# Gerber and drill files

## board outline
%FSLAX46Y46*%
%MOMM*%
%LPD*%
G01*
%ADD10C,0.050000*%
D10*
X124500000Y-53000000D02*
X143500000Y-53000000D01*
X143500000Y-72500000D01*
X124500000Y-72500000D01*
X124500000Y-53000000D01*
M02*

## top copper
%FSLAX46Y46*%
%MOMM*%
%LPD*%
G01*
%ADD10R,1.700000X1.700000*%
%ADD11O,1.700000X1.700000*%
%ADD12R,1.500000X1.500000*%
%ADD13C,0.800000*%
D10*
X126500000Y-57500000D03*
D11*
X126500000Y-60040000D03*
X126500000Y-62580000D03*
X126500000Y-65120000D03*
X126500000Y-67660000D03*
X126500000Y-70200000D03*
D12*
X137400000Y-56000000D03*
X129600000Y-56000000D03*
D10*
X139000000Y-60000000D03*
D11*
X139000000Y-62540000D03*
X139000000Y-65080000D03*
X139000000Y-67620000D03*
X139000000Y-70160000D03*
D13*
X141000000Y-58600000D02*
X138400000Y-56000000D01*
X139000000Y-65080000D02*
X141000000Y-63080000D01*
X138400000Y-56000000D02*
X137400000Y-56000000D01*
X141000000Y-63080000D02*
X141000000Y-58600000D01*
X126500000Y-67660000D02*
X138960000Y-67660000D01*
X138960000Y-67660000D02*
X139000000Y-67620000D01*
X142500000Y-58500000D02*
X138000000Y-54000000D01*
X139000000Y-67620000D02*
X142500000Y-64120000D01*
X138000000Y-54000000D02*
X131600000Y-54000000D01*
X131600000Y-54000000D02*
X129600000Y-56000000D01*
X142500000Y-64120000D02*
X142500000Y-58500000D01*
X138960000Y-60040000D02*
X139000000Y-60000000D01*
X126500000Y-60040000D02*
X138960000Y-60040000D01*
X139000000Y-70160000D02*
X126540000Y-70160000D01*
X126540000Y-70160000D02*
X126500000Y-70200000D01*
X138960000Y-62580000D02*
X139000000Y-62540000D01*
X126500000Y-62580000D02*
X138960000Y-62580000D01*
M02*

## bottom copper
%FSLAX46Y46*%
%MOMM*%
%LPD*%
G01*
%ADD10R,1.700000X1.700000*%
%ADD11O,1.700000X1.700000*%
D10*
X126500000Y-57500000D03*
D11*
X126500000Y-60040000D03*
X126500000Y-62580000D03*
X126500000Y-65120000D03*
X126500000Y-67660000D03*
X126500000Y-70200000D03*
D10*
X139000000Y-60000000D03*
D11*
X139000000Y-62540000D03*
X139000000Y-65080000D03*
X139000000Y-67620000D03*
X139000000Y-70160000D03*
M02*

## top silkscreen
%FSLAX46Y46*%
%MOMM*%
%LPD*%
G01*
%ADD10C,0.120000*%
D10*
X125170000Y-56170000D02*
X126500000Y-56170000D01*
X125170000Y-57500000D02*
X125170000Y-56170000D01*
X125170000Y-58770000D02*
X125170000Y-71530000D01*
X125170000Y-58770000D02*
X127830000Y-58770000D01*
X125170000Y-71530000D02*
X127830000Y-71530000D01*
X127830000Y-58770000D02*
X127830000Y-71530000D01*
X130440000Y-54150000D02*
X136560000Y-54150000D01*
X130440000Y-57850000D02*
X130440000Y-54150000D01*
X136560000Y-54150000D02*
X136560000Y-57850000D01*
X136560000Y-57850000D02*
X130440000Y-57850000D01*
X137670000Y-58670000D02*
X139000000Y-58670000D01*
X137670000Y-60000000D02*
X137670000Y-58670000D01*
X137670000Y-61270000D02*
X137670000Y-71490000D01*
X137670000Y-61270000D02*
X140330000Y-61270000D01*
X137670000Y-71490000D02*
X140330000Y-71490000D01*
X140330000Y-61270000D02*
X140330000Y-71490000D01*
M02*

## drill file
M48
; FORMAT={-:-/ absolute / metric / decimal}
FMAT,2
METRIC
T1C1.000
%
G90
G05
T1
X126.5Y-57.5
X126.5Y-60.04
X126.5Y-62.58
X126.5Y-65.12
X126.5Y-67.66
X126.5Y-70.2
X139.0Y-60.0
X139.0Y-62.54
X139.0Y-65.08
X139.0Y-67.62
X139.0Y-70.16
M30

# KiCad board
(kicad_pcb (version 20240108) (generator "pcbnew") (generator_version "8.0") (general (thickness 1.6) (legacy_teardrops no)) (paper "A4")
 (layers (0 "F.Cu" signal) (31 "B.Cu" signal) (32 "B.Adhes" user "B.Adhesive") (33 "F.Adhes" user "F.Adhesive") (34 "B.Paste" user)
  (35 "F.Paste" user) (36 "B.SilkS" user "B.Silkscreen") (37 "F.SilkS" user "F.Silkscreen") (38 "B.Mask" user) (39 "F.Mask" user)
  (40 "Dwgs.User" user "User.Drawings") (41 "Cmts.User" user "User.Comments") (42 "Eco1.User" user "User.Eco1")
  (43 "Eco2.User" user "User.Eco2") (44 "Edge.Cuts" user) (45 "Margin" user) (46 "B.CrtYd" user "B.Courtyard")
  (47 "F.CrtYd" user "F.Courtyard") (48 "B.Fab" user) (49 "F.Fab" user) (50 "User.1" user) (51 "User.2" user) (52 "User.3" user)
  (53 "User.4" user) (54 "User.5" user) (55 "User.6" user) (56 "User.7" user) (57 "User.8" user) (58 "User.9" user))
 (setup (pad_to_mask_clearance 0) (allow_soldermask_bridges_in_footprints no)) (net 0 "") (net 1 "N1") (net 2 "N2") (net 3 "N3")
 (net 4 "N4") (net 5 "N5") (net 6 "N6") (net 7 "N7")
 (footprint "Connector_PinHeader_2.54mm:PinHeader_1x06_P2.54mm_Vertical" (layer "F.Cu") (at 126.5 57.5)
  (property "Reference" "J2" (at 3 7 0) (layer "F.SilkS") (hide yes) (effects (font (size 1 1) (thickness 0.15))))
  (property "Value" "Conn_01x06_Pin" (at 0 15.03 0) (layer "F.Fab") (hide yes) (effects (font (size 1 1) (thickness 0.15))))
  (fp_line (start -1.33 -1.33) (end 0 -1.33) (stroke (width 0.12) (type solid)) (layer "F.SilkS"))
  (fp_line (start -1.33 0) (end -1.33 -1.33) (stroke (width 0.12) (type solid)) (layer "F.SilkS"))
  (fp_line (start -1.33 1.27) (end -1.33 14.03) (stroke (width 0.12) (type solid)) (layer "F.SilkS"))
  (fp_line (start -1.33 1.27) (end 1.33 1.27) (stroke (width 0.12) (type solid)) (layer "F.SilkS"))
  (fp_line (start -1.33 14.03) (end 1.33 14.03) (stroke (width 0.12) (type solid)) (layer "F.SilkS"))
  (fp_line (start 1.33 1.27) (end 1.33 14.03) (stroke (width 0.12) (type solid)) (layer "F.SilkS"))
  (pad "1" thru_hole rect (at 0 0) (size 1.7 1.7) (drill 1) (layers "*.Cu" "*.Mask") (remove_unused_layers no) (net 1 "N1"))
  (pad "2" thru_hole oval (at 0 2.54) (size 1.7 1.7) (drill 1) (layers "*.Cu" "*.Mask") (remove_unused_layers no) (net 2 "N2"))
  (pad "3" thru_hole oval (at 0 5.08) (size 1.7 1.7) (drill 1) (layers "*.Cu" "*.Mask") (remove_unused_layers no) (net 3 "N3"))
  (pad "4" thru_hole oval (at 0 7.62) (size 1.7 1.7) (drill 1) (layers "*.Cu" "*.Mask") (remove_unused_layers no) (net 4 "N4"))
  (pad "5" thru_hole oval (at 0 10.16) (size 1.7 1.7) (drill 1) (layers "*.Cu" "*.Mask") (remove_unused_layers no) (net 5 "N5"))
  (pad "6" thru_hole oval (at 0 12.7) (size 1.7 1.7) (drill 1) (layers "*.Cu" "*.Mask") (remove_unused_layers no) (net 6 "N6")))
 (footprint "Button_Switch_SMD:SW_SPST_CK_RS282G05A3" (layer "F.Cu") (at 133.5 56 180)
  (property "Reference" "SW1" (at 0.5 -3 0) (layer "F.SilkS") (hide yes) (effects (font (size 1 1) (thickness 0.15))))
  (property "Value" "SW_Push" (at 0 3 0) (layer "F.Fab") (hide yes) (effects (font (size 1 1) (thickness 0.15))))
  (fp_line (start 3.06 1.85) (end -3.06 1.85) (stroke (width 0.12) (type solid)) (layer "F.SilkS"))
  (fp_line (start 3.06 -1.85) (end 3.06 1.85) (stroke (width 0.12) (type solid)) (layer "F.SilkS"))
  (fp_line (start -3.06 1.85) (end -3.06 -1.85) (stroke (width 0.12) (type solid)) (layer "F.SilkS"))
  (fp_line (start -3.06 -1.85) (end 3.06 -1.85) (stroke (width 0.12) (type solid)) (layer "F.SilkS"))
  (pad "1" smd rect (at -3.9 0 180) (size 1.5 1.5) (layers "F.Cu" "F.Paste" "F.Mask") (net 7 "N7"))
  (pad "2" smd rect (at 3.9 0 180) (size 1.5 1.5) (layers "F.Cu" "F.Paste" "F.Mask") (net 5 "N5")))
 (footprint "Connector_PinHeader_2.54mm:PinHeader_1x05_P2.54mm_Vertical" (layer "F.Cu") (at 139 60)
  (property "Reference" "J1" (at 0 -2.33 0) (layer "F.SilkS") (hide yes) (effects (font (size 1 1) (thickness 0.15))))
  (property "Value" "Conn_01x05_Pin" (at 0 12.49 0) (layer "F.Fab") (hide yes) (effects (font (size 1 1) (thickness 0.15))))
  (fp_line (start -1.33 -1.33) (end 0 -1.33) (stroke (width 0.12) (type solid)) (layer "F.SilkS"))
  (fp_line (start -1.33 0) (end -1.33 -1.33) (stroke (width 0.12) (type solid)) (layer "F.SilkS"))
  (fp_line (start -1.33 1.27) (end -1.33 11.49) (stroke (width 0.12) (type solid)) (layer "F.SilkS"))
  (fp_line (start -1.33 1.27) (end 1.33 1.27) (stroke (width 0.12) (type solid)) (layer "F.SilkS"))
  (fp_line (start -1.33 11.49) (end 1.33 11.49) (stroke (width 0.12) (type solid)) (layer "F.SilkS"))
  (fp_line (start 1.33 1.27) (end 1.33 11.49) (stroke (width 0.12) (type solid)) (layer "F.SilkS"))
  (pad "1" thru_hole rect (at 0 0) (size 1.7 1.7) (drill 1) (layers "*.Cu" "*.Mask") (remove_unused_layers no) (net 2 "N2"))
  (pad "2" thru_hole oval (at 0 2.54) (size 1.7 1.7) (drill 1) (layers "*.Cu" "*.Mask") (remove_unused_layers no) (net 3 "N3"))
  (pad "3" thru_hole oval (at 0 5.08) (size 1.7 1.7) (drill 1) (layers "*.Cu" "*.Mask") (remove_unused_layers no) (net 7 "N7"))
  (pad "4" thru_hole oval (at 0 7.62) (size 1.7 1.7) (drill 1) (layers "*.Cu" "*.Mask") (remove_unused_layers no) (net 5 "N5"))
  (pad "5" thru_hole oval (at 0 10.16) (size 1.7 1.7) (drill 1) (layers "*.Cu" "*.Mask") (remove_unused_layers no) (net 6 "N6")))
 (gr_rect (start 124.5 53) (end 143.5 72.5) (stroke (width 0.05) (type default)) (fill none) (layer "Edge.Cuts"))
 (segment (start 141 58.6) (end 138.4 56) (width 0.8) (layer "F.Cu") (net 7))
 (segment (start 139 65.08) (end 141 63.08) (width 0.8) (layer "F.Cu") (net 7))
 (segment (start 138.4 56) (end 137.4 56) (width 0.8) (layer "F.Cu") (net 7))
 (segment (start 141 63.08) (end 141 58.6) (width 0.8) (layer "F.Cu") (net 7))
 (segment (start 126.5 67.66) (end 138.96 67.66) (width 0.8) (layer "F.Cu") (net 5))
 (segment (start 138.96 67.66) (end 139 67.62) (width 0.8) (layer "F.Cu") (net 5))
 (segment (start 142.5 58.5) (end 138 54) (width 0.8) (layer "F.Cu") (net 5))
 (segment (start 139 67.62) (end 142.5 64.12) (width 0.8) (layer "F.Cu") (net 5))
 (segment (start 138 54) (end 131.6 54) (width 0.8) (layer "F.Cu") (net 5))
 (segment (start 131.6 54) (end 129.6 56) (width 0.8) (layer "F.Cu") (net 5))
 (segment (start 142.5 64.12) (end 142.5 58.5) (width 0.8) (layer "F.Cu") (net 5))
 (segment (start 138.96 60.04) (end 139 60) (width 0.8) (layer "F.Cu") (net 2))
 (segment (start 126.5 60.04) (end 138.96 60.04) (width 0.8) (layer "F.Cu") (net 2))
 (segment (start 139 70.16) (end 126.54 70.16) (width 0.8) (layer "F.Cu") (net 6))
 (segment (start 126.54 70.16) (end 126.5 70.2) (width 0.8) (layer "F.Cu") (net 6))
 (segment (start 138.96 62.58) (end 139 62.54) (width 0.8) (layer "F.Cu") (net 3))
 (segment (start 126.5 62.58) (end 138.96 62.58) (width 0.8) (layer "F.Cu") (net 3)))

